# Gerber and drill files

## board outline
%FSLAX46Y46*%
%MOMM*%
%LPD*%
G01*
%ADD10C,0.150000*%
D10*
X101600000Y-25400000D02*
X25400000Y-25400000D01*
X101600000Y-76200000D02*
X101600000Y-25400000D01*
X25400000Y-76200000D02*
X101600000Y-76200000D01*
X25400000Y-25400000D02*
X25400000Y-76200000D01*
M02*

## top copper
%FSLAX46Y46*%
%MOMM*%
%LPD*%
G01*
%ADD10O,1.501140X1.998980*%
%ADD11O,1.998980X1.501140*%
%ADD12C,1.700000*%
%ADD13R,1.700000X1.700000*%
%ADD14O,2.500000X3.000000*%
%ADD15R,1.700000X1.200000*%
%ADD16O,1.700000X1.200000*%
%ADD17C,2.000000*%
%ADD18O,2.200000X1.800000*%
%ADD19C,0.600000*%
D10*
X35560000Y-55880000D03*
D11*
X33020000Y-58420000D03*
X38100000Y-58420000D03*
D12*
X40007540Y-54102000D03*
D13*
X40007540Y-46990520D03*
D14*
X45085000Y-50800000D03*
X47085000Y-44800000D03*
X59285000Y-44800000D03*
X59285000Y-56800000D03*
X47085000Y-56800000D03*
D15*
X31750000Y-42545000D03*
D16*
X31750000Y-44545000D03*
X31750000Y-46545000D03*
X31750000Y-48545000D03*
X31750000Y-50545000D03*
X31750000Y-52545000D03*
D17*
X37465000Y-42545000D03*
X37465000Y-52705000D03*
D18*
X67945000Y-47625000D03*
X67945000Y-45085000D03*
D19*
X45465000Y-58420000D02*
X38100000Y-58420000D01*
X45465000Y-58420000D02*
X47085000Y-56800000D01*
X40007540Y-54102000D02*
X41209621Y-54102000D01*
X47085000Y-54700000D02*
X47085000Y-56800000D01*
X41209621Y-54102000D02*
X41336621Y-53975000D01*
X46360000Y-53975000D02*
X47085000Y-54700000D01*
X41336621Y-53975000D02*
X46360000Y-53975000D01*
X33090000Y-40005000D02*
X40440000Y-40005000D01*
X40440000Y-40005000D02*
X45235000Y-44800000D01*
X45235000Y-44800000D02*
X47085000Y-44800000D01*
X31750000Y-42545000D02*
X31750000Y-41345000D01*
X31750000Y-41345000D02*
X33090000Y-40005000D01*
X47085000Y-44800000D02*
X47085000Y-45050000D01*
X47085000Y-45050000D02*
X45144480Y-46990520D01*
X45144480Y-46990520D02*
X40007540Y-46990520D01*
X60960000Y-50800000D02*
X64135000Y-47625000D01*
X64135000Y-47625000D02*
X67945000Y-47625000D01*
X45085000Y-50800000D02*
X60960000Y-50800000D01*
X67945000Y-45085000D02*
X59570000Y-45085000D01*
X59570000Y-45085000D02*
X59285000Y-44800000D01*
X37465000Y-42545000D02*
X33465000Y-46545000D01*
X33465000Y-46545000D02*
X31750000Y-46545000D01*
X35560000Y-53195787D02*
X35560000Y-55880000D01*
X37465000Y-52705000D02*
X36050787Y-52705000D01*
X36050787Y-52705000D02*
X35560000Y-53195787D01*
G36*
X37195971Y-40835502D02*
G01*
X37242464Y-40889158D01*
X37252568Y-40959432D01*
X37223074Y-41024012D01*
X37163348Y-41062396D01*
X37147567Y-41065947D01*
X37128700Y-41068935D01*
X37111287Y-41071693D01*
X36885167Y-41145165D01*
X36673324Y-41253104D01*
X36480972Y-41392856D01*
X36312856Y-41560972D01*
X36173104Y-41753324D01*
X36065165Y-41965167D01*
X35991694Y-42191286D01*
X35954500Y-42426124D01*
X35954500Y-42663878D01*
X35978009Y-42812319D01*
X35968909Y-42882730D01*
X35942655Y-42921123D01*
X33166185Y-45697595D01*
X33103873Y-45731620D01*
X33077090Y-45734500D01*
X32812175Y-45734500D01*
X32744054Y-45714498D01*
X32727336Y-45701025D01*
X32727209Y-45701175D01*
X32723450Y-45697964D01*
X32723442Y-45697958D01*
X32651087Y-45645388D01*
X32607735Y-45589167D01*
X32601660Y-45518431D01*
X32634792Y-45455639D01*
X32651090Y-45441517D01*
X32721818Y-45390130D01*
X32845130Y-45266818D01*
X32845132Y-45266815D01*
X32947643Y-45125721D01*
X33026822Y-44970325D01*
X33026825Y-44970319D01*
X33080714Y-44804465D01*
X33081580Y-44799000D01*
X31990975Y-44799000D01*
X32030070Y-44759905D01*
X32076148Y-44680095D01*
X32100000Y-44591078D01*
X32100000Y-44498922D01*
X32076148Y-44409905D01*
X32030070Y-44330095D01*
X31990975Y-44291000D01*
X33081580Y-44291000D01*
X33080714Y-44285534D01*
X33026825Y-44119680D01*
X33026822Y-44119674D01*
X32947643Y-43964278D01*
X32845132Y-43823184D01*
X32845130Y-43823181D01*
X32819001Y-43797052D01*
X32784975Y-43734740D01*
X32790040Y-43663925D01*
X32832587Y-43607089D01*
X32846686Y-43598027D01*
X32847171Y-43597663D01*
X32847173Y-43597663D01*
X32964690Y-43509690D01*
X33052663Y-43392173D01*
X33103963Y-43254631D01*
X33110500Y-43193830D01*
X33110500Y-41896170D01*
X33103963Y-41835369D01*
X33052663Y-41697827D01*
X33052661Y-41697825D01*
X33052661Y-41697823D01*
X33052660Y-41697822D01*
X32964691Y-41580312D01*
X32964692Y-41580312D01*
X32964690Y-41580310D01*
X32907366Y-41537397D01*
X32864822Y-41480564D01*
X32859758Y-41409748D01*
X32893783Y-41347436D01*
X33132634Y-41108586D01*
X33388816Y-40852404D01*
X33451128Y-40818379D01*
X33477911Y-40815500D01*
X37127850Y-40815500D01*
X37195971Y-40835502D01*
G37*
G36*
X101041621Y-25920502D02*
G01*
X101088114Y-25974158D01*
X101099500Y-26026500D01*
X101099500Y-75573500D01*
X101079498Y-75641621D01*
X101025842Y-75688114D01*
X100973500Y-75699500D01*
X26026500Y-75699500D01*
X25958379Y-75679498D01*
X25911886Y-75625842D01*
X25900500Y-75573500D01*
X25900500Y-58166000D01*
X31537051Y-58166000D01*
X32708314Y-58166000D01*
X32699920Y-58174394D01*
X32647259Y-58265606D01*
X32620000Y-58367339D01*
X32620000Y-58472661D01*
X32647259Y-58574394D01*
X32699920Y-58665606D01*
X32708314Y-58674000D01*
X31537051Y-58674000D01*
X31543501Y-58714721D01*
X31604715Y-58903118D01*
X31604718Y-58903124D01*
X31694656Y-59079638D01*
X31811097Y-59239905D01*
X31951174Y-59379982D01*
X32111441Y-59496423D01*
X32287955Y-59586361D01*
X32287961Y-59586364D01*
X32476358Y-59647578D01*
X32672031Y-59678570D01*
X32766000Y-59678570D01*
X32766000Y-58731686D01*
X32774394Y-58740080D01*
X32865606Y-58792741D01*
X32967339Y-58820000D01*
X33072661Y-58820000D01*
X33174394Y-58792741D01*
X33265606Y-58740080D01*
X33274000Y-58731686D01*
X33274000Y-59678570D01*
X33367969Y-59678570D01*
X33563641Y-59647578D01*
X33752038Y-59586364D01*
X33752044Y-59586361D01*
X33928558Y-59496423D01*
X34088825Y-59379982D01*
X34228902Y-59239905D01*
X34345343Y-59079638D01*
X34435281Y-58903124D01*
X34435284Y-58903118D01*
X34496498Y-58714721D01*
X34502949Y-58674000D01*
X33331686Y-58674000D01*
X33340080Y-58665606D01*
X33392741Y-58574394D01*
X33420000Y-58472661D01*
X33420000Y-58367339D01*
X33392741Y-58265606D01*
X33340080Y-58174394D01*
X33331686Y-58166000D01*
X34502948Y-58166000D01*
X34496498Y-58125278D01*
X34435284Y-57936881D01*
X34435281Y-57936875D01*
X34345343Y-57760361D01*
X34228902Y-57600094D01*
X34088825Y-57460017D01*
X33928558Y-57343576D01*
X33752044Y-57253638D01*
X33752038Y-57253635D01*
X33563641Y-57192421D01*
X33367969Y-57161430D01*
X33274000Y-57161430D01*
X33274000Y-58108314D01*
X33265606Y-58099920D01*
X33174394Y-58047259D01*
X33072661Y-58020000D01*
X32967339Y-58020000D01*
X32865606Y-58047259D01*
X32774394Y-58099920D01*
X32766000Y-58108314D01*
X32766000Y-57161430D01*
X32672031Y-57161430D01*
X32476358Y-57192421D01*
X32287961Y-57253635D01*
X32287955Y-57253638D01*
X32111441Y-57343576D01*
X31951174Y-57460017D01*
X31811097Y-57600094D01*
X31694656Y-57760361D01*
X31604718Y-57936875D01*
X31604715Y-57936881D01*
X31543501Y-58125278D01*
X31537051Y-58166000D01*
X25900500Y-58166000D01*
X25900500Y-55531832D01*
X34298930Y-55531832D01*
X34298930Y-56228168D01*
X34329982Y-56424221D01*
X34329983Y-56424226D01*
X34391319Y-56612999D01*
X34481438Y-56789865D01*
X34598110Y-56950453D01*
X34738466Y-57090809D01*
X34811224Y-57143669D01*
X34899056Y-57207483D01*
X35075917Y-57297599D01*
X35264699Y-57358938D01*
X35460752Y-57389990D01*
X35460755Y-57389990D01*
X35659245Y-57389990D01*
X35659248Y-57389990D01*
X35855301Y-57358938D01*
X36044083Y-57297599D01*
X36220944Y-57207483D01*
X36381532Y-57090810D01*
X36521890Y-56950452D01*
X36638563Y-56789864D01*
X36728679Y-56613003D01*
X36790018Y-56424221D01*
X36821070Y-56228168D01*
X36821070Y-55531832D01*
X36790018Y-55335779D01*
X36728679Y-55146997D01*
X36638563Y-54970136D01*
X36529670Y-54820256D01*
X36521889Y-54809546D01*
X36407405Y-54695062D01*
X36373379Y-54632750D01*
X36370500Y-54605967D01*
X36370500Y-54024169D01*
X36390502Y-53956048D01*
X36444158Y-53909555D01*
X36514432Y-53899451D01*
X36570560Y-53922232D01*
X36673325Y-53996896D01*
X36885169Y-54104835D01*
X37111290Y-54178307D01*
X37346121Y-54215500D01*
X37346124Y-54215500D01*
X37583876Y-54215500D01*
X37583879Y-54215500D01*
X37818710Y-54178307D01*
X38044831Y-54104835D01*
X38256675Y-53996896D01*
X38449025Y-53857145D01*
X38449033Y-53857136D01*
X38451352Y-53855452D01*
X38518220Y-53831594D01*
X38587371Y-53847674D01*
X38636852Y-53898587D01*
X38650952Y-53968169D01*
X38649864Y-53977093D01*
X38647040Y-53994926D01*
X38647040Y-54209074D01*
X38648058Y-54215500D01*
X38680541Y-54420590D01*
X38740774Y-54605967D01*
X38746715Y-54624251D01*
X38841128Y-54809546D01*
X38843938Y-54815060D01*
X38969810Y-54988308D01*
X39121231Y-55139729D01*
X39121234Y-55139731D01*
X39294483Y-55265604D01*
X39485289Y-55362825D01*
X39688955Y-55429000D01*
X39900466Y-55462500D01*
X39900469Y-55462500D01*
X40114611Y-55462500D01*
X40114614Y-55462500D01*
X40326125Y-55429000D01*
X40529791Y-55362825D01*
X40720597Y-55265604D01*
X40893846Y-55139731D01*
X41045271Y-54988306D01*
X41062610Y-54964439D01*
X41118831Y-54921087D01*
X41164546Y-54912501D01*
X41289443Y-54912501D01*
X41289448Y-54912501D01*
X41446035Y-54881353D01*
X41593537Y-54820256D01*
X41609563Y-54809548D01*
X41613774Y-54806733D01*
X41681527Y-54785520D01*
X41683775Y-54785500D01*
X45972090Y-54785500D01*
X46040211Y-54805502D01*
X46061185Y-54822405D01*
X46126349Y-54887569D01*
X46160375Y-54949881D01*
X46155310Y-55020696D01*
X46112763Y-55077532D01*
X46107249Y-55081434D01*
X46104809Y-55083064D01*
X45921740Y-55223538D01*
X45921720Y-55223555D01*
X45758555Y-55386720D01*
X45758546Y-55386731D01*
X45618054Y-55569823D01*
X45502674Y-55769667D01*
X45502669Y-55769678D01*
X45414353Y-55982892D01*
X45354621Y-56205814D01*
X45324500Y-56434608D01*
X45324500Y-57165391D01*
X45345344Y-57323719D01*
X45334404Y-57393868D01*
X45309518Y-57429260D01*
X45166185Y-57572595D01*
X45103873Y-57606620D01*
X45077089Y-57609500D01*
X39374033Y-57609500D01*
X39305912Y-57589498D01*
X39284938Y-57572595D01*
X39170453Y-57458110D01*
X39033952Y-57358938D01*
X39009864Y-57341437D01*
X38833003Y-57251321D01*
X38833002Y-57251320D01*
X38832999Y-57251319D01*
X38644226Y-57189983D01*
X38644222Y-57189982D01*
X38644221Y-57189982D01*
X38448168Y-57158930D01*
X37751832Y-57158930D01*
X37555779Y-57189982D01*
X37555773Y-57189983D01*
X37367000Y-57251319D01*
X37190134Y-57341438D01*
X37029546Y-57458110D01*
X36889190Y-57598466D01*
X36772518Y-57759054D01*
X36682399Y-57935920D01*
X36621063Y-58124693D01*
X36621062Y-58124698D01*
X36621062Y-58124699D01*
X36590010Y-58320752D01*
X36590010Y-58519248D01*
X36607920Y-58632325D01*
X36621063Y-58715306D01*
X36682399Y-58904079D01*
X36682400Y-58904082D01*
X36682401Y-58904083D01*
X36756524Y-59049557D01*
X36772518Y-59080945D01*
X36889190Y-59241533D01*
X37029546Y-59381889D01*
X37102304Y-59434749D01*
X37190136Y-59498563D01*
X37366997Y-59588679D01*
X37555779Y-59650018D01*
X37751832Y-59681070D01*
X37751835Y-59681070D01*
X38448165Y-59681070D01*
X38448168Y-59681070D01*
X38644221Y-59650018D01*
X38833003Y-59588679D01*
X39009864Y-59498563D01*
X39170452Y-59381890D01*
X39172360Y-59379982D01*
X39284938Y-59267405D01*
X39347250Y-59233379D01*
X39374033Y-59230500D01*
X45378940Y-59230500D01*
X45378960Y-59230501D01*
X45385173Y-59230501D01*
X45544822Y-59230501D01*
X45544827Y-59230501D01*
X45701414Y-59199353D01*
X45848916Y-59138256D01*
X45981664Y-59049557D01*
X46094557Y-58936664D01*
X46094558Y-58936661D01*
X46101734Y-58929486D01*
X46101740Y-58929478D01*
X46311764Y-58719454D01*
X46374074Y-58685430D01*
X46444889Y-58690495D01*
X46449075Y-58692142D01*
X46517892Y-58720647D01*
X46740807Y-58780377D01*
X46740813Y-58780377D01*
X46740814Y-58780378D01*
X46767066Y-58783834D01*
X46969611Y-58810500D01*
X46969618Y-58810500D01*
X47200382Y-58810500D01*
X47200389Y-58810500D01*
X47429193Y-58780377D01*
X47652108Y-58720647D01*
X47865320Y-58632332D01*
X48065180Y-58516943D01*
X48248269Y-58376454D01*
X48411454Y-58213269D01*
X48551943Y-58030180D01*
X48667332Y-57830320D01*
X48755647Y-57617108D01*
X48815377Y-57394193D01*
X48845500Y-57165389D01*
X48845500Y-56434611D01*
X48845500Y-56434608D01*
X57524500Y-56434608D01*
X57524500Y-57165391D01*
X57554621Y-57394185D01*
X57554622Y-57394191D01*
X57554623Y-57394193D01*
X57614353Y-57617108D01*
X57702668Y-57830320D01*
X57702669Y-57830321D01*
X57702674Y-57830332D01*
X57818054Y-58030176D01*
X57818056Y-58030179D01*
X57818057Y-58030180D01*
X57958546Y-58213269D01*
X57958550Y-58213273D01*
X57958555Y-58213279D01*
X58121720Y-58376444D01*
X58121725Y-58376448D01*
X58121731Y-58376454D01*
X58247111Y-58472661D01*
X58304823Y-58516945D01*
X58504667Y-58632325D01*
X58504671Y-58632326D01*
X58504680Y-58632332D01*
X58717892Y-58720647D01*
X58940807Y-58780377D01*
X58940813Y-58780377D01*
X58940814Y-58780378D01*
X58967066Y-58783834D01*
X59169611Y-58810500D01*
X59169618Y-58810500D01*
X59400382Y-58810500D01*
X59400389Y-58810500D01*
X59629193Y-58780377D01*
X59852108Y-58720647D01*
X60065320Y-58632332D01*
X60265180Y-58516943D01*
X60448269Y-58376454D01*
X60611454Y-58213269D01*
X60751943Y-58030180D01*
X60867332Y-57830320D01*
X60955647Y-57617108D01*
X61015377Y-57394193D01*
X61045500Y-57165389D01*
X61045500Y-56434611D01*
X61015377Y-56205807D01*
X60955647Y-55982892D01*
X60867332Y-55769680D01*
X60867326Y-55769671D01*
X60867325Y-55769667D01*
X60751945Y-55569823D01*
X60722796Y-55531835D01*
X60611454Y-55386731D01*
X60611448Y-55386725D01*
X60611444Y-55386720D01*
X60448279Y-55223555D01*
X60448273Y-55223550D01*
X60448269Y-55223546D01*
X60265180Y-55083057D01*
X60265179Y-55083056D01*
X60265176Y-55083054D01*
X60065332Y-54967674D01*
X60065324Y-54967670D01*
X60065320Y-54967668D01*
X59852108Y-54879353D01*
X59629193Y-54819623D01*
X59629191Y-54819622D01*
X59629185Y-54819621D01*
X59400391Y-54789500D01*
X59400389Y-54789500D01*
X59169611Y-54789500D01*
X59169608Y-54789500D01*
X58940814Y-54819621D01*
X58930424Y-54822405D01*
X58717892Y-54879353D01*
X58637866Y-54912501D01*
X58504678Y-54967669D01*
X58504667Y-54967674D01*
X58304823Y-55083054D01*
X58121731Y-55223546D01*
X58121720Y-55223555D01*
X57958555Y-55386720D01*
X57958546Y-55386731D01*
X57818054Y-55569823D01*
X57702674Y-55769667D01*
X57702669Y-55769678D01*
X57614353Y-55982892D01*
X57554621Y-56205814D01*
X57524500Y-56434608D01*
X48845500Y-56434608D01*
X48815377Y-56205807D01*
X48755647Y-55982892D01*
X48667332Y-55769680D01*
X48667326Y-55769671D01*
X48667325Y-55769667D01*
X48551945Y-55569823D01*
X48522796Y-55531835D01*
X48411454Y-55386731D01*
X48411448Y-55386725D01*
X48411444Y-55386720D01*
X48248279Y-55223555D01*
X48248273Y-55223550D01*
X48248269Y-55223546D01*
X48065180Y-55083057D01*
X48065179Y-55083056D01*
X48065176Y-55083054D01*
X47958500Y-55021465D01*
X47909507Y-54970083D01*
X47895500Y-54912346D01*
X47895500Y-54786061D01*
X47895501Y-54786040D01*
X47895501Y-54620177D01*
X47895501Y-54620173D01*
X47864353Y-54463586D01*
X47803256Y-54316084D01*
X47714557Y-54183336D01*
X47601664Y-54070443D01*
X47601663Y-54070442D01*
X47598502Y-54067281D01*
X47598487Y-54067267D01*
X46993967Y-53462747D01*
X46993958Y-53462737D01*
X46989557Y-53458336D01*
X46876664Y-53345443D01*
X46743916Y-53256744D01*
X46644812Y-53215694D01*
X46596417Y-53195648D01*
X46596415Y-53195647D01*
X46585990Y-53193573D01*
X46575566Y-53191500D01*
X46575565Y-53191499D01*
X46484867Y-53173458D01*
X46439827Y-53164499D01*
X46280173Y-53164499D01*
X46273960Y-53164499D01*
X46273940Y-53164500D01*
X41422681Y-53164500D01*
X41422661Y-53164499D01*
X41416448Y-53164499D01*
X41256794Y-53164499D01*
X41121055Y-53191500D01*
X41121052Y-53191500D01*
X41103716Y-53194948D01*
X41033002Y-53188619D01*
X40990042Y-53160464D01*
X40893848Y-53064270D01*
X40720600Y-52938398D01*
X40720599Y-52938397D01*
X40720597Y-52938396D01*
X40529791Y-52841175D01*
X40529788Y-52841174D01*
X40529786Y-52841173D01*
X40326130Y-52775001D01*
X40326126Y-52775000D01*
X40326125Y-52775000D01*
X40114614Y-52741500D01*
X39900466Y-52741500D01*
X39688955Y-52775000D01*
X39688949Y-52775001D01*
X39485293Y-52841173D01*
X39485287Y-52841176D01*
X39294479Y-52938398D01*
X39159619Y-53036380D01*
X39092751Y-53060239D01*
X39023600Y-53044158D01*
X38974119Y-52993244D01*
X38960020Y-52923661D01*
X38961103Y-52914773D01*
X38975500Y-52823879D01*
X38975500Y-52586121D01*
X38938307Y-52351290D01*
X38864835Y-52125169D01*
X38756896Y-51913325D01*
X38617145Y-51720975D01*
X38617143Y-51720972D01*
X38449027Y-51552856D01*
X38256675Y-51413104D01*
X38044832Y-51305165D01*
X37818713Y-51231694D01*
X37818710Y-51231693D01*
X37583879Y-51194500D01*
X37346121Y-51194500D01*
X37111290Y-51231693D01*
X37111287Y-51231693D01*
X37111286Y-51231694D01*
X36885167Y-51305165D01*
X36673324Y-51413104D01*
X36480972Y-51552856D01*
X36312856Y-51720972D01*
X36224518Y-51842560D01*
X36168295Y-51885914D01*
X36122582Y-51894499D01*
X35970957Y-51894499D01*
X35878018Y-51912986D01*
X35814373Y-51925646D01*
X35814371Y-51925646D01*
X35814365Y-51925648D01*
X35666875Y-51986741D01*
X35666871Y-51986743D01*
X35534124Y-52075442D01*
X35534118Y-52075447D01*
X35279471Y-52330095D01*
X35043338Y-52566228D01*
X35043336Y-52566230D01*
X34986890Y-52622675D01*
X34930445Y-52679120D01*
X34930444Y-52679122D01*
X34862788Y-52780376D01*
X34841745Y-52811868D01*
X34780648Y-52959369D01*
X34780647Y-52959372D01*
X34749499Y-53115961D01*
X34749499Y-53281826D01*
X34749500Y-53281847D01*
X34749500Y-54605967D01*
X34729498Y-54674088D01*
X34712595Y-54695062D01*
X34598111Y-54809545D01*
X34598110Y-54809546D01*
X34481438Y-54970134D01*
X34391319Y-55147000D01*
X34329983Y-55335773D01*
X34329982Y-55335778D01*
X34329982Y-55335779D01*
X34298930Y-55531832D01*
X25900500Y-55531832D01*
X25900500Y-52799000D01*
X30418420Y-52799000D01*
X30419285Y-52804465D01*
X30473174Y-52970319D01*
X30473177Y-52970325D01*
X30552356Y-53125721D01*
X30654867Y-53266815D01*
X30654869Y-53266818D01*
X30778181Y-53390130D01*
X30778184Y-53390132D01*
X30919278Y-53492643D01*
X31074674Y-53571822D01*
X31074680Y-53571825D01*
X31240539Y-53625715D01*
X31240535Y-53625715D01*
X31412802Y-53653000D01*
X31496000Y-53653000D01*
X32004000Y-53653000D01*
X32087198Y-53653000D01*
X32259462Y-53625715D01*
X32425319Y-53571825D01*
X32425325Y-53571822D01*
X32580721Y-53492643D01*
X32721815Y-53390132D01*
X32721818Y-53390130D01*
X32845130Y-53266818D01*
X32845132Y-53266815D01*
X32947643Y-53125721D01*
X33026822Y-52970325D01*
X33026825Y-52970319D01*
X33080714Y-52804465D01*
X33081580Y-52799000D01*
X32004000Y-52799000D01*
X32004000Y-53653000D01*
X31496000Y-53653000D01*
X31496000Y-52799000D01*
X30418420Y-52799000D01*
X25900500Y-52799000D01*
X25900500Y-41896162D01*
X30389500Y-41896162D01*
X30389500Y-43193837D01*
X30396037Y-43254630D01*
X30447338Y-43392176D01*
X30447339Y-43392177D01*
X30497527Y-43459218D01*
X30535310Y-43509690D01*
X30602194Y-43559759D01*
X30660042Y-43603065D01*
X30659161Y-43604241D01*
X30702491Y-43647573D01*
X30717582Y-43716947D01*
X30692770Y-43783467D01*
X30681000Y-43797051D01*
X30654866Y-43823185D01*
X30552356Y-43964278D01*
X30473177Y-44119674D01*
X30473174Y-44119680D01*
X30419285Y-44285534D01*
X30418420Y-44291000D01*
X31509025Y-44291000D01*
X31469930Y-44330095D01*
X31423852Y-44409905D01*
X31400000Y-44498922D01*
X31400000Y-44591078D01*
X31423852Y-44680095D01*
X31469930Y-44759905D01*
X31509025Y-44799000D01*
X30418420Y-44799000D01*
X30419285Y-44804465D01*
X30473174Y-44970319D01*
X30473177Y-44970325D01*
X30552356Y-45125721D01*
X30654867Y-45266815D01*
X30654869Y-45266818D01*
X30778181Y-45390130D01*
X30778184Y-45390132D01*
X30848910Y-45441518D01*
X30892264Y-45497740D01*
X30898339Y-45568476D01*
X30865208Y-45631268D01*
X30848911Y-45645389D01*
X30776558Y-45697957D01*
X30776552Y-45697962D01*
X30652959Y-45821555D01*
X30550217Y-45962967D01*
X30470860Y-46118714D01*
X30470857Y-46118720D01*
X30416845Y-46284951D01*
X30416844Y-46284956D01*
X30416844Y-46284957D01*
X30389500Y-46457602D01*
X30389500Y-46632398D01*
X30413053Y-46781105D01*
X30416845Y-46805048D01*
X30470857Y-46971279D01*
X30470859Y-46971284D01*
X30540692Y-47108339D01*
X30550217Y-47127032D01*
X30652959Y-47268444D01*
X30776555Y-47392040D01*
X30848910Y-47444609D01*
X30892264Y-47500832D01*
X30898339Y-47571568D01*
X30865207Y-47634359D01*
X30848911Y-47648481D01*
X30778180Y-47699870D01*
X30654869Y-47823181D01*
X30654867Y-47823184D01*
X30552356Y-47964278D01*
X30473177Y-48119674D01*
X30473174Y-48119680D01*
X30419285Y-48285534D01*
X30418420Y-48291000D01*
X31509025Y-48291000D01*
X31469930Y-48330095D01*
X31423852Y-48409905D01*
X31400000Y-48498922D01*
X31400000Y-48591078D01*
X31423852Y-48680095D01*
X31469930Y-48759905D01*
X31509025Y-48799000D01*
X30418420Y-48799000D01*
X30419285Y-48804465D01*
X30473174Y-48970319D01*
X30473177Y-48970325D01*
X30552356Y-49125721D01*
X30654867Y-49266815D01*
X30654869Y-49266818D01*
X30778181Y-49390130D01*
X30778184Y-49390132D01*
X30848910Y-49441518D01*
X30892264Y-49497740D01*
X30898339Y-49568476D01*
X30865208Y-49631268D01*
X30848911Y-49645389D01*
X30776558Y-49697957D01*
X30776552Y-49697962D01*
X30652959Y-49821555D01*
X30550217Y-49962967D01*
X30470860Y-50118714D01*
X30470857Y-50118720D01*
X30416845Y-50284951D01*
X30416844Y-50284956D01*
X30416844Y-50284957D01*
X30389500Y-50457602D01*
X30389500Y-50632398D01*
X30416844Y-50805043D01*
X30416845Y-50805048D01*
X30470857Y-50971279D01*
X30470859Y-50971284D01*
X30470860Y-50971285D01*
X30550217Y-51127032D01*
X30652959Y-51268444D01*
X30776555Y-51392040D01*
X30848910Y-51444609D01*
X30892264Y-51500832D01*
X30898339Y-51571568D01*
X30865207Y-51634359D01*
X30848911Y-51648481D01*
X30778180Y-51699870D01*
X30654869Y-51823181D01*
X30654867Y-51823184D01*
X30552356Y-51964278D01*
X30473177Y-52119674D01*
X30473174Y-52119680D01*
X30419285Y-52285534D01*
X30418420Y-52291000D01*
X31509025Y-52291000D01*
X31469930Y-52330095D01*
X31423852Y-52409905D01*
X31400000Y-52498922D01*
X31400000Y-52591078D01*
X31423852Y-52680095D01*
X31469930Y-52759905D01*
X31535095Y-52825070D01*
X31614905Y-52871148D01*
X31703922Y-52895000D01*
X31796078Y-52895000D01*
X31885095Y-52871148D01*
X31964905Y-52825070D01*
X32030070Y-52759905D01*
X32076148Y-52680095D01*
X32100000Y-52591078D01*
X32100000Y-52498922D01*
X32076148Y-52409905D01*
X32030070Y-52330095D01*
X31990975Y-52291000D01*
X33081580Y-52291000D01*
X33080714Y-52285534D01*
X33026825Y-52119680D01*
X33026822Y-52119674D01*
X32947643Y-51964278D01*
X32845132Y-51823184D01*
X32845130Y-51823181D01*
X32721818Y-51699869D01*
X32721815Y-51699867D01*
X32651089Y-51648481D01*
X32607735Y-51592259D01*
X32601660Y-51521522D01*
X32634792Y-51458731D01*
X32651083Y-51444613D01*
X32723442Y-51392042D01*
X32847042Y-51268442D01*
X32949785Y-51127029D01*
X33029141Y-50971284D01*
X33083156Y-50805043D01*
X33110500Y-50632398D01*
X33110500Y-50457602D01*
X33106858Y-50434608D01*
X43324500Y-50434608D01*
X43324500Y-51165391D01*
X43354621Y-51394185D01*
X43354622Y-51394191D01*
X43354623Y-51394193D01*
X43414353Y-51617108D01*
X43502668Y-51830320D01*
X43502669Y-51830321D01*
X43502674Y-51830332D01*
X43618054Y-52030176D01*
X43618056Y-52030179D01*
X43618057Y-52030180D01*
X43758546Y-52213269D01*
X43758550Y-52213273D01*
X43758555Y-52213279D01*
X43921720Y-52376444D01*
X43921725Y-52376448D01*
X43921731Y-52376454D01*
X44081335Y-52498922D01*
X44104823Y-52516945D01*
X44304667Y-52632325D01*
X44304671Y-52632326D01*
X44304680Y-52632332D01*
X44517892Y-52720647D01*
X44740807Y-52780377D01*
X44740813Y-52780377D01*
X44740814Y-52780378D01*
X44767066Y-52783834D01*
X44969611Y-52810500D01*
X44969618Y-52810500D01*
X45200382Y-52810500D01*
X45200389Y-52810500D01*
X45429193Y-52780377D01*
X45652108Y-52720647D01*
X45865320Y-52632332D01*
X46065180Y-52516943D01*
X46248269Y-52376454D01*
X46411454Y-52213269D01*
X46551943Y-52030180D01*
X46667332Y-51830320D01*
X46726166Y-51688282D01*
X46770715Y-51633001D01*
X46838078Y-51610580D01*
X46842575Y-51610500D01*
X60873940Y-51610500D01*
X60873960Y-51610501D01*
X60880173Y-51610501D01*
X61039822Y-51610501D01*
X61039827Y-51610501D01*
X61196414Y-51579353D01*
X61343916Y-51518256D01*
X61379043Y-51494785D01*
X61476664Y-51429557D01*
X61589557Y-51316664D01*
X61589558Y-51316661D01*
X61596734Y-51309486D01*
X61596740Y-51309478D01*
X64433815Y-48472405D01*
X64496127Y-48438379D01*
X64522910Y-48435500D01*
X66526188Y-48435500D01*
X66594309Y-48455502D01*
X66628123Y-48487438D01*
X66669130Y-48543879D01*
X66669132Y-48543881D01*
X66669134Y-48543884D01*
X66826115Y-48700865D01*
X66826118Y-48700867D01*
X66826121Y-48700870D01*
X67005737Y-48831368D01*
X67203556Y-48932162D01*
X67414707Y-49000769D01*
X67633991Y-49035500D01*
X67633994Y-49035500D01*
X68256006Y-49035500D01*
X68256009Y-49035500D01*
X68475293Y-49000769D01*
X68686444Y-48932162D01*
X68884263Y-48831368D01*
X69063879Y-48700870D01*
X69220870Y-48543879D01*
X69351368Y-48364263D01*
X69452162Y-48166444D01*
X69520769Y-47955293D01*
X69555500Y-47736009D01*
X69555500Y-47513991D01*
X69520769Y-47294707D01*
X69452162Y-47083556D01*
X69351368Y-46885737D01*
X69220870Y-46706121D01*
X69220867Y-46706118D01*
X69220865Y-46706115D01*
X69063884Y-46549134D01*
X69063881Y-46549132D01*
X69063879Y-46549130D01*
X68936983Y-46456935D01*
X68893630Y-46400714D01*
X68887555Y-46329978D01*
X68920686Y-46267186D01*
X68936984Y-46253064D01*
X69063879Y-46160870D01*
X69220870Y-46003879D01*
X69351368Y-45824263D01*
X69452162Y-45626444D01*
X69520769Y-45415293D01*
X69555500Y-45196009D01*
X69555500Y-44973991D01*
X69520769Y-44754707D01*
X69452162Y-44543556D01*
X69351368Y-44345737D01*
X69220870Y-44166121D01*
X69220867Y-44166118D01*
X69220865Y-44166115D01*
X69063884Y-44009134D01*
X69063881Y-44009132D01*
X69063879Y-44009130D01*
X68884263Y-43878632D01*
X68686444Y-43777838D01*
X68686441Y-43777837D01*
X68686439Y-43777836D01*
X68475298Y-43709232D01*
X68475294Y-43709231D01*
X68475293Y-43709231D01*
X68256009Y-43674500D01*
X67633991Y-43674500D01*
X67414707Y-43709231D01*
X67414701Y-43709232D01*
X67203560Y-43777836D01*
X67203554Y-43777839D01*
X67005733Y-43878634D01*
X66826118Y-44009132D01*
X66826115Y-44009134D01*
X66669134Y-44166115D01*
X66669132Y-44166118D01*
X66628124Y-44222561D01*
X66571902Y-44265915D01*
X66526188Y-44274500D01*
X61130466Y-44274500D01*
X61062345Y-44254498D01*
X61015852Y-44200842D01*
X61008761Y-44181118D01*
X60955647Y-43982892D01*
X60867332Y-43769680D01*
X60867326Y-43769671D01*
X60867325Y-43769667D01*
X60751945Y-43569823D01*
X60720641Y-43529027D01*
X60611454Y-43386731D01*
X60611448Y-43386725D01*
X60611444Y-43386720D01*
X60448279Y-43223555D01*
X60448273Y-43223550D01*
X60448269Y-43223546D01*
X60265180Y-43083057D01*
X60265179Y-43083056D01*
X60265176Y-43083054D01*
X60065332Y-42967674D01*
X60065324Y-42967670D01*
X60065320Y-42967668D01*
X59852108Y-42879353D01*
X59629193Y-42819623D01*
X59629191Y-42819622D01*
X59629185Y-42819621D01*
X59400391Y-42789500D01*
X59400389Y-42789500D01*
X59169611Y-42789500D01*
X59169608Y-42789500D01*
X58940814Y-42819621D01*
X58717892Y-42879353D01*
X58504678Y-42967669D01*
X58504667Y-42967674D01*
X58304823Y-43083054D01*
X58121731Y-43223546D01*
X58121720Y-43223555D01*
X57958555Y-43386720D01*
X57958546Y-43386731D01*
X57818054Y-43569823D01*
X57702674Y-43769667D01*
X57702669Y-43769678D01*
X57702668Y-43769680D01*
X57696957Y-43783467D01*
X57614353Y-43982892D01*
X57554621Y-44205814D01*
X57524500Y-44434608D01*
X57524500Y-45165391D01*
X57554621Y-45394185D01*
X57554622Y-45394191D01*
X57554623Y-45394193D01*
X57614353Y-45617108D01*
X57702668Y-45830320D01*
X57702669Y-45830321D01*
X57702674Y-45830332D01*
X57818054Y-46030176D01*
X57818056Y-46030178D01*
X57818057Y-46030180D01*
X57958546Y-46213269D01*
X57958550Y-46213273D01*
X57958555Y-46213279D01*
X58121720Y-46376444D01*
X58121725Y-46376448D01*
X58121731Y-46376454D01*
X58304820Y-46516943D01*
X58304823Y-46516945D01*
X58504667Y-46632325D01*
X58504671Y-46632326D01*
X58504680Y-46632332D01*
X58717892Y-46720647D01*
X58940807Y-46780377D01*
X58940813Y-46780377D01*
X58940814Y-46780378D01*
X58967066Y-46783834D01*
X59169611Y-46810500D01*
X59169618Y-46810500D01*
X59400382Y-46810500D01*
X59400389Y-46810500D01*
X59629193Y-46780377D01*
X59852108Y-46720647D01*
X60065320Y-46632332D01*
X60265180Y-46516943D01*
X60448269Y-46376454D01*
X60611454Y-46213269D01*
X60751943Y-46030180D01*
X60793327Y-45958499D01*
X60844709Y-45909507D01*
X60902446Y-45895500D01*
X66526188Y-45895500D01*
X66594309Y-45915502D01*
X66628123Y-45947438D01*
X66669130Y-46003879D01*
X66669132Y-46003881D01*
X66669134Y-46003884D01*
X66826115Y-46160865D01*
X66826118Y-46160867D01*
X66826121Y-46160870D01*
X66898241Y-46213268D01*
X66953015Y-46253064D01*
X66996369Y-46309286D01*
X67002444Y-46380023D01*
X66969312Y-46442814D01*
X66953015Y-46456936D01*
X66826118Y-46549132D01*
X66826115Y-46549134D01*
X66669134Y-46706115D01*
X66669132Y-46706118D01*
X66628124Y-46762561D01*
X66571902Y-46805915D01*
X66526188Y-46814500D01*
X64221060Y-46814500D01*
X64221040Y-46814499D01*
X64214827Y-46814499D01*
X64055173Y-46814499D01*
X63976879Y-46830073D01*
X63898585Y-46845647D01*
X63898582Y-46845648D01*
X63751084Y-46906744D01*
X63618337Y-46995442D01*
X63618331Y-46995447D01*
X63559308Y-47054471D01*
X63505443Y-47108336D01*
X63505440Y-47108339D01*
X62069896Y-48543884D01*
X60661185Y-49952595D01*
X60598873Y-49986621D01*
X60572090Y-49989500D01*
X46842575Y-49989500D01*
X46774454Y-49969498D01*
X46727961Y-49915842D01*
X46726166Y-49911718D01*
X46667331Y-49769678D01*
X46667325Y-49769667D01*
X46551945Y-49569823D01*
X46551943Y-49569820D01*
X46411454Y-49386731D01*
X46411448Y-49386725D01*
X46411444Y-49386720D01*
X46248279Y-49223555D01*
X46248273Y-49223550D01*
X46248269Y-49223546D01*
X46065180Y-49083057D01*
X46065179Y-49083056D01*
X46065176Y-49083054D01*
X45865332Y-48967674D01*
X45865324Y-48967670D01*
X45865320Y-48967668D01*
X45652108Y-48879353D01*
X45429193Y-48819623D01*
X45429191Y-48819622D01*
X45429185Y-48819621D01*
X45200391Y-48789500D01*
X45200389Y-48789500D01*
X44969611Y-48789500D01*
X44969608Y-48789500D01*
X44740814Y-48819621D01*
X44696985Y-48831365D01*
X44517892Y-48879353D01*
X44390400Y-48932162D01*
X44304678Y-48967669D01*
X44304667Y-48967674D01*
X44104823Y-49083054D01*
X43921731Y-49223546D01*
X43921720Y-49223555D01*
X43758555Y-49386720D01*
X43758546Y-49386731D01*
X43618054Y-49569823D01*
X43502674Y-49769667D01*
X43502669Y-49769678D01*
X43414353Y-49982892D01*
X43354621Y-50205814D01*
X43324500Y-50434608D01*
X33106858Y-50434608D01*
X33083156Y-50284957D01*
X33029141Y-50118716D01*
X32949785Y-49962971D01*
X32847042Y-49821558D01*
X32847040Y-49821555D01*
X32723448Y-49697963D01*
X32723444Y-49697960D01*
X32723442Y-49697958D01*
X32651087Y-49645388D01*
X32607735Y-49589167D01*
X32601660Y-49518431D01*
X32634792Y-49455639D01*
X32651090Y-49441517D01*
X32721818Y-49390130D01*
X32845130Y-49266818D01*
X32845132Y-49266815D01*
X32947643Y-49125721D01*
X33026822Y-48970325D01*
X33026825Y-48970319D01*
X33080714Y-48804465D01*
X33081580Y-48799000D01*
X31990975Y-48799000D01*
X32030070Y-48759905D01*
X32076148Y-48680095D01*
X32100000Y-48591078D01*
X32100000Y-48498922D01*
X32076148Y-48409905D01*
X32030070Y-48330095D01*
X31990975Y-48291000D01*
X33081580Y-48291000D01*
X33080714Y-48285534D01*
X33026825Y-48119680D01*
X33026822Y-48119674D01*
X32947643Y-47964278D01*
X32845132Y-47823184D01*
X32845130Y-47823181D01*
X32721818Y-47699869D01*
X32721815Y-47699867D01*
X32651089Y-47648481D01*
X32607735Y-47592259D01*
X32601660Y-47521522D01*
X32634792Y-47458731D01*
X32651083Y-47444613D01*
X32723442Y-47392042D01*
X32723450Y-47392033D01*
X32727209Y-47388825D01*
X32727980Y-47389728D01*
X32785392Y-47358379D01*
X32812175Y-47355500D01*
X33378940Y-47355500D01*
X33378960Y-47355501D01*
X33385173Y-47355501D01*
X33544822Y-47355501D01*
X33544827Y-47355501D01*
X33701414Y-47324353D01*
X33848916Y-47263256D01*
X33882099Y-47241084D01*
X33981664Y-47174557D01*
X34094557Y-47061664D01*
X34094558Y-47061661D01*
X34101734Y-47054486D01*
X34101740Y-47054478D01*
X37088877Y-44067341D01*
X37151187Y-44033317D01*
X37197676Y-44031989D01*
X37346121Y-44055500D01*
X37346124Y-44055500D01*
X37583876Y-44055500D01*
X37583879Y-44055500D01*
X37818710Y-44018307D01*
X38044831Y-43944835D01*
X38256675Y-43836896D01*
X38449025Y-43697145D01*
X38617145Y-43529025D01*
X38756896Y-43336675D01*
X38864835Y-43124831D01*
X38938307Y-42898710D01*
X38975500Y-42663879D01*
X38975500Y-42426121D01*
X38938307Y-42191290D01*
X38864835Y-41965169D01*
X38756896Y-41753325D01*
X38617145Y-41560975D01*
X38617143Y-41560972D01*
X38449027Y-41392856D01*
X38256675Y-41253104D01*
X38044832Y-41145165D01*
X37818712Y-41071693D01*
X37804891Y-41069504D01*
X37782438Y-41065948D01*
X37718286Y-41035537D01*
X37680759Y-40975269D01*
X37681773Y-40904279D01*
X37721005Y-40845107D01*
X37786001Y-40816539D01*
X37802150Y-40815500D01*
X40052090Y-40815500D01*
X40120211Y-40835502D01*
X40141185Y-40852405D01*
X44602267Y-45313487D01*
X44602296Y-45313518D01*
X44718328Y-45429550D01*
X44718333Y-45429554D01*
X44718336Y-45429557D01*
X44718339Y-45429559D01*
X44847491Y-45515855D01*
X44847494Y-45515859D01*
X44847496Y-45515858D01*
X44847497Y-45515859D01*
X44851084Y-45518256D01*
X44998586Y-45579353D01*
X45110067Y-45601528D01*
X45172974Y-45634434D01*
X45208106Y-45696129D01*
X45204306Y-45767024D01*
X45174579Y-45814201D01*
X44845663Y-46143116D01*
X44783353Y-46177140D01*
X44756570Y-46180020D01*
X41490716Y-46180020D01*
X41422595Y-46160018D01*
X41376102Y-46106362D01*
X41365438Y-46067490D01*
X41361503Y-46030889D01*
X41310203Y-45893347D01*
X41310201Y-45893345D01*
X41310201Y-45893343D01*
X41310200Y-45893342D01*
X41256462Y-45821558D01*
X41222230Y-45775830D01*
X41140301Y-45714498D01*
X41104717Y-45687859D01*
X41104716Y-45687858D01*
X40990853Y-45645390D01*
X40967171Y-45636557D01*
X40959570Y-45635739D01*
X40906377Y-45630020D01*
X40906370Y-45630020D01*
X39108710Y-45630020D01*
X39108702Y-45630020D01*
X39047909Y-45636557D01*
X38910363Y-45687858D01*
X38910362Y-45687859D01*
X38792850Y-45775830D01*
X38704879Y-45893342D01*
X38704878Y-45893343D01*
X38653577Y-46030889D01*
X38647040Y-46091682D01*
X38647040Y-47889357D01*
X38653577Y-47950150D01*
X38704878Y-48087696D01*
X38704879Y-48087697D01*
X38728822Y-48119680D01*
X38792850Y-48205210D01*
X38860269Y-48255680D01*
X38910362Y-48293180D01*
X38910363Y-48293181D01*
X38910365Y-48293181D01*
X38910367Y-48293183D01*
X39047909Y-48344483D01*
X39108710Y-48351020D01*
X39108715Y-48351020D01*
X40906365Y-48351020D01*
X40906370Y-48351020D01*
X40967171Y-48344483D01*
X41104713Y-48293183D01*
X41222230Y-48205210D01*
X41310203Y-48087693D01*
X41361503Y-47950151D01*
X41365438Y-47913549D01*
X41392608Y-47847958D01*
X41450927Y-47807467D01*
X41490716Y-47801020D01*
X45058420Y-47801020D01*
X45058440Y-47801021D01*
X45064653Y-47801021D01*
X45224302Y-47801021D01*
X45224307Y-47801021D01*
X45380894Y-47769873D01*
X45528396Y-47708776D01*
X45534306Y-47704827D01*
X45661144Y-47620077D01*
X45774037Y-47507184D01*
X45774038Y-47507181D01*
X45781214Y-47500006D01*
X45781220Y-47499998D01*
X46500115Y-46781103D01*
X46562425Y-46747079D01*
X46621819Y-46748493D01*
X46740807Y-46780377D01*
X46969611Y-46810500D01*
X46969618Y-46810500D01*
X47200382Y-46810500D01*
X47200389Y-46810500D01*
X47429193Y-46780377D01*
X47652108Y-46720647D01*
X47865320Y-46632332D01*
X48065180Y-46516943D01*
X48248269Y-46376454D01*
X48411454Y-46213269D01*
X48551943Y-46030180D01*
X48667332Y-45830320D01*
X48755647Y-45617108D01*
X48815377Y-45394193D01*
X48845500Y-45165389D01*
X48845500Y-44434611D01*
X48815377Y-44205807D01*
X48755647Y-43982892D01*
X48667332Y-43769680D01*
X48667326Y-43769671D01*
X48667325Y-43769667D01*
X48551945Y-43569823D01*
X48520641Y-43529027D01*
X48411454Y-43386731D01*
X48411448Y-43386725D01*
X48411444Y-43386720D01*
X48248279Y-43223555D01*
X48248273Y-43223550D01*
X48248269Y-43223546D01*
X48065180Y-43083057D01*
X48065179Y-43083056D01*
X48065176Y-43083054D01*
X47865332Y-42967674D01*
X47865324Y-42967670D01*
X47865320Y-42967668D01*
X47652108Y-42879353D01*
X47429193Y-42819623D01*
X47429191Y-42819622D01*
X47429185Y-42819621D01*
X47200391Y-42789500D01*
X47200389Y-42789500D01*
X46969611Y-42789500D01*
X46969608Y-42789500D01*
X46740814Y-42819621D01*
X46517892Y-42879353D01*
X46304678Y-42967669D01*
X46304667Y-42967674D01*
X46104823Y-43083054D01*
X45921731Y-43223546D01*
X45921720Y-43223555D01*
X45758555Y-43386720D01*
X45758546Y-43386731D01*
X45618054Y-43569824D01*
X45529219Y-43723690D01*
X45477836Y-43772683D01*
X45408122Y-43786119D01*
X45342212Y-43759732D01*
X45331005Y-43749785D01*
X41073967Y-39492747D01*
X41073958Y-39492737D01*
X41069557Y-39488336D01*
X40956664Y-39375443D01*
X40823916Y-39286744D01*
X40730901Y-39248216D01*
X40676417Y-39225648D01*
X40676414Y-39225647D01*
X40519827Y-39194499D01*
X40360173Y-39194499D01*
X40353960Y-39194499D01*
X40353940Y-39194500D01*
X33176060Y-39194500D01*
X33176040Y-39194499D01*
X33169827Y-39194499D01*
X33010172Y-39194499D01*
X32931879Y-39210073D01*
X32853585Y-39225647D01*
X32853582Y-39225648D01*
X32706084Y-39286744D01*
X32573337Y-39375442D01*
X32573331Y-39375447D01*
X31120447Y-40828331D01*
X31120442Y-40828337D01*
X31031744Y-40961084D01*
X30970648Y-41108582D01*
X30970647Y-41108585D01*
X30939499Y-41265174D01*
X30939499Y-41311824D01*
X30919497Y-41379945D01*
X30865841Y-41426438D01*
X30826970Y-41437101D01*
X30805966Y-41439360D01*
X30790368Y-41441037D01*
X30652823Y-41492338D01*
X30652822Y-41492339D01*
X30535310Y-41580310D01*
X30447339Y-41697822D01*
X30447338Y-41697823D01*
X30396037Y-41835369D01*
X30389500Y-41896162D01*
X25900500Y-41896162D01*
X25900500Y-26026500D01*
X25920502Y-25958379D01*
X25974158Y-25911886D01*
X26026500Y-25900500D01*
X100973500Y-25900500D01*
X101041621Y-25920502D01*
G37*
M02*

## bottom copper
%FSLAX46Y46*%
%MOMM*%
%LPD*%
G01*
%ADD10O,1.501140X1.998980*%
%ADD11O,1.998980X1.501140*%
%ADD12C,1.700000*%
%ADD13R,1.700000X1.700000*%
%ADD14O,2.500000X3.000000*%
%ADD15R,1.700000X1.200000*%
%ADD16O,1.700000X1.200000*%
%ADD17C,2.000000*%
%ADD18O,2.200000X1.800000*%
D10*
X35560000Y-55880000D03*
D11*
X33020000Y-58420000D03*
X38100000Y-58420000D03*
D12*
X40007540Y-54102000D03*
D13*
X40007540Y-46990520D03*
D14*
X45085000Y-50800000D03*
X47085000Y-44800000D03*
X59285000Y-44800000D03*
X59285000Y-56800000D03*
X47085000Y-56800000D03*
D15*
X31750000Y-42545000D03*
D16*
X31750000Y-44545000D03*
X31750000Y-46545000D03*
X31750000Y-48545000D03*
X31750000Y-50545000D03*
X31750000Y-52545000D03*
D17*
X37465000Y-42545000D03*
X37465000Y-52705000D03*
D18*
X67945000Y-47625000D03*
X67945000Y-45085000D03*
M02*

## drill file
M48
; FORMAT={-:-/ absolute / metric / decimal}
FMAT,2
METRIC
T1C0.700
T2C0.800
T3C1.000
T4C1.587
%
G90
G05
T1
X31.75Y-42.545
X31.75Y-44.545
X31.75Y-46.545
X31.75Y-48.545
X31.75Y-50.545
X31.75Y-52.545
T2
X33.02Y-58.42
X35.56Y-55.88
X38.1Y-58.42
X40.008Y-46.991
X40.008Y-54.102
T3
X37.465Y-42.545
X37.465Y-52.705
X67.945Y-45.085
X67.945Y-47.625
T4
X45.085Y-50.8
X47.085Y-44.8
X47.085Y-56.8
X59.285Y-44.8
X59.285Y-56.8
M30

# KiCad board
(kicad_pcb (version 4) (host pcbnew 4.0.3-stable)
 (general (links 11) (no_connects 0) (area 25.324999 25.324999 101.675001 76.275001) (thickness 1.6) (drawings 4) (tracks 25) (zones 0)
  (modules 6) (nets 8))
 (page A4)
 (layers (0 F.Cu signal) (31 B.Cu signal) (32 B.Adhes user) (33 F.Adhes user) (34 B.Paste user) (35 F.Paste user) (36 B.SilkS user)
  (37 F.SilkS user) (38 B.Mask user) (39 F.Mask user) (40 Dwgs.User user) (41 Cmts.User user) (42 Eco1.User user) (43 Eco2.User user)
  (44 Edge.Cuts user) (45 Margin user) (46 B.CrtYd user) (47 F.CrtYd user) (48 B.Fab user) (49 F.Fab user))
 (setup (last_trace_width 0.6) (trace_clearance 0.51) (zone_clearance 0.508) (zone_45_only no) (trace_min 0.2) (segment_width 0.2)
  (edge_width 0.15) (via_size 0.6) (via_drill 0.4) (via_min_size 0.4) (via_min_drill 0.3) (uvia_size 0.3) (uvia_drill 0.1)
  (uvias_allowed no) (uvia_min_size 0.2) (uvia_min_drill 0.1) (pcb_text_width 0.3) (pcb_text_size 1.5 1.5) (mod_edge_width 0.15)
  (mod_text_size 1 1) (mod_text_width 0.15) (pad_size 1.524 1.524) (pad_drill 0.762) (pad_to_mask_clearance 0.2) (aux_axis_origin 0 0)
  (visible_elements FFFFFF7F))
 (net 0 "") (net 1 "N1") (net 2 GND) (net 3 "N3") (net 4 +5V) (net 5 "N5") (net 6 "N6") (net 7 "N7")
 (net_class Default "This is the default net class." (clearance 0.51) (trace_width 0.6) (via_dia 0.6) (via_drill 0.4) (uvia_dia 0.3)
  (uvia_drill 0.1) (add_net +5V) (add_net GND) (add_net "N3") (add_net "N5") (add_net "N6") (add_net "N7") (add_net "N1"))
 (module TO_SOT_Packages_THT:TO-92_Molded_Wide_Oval (layer F.Cu) (at 33.02 58.42)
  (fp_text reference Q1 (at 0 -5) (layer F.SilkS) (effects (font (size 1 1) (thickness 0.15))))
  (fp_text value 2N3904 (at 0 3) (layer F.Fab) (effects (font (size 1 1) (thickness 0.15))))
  (pad 2 thru_hole oval (at 2.54 -2.54 90) (size 1.99898 1.50114) (drill 0.8) (layers *.Cu *.Mask F.SilkS) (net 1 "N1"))
  (pad 1 thru_hole oval (at 0 0 90) (size 1.50114 1.99898) (drill 0.8) (layers *.Cu *.Mask F.SilkS) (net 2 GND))
  (pad 3 thru_hole oval (at 5.08 0 90) (size 1.50114 1.99898) (drill 0.8) (layers *.Cu *.Mask F.SilkS) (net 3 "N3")))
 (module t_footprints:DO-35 (layer F.Cu) (at 40.005 46.99 270)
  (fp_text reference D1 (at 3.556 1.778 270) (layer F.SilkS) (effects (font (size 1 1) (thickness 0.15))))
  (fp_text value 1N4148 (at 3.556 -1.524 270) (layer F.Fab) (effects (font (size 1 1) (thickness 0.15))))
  (pad 2 thru_hole circle (at 7.112 -0.00254 90) (size 1.7 1.7) (drill 0.8) (layers *.Cu *.Mask F.SilkS) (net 3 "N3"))
  (pad 1 thru_hole rect (at 0.00052 -0.00254 90) (size 1.7 1.7) (drill 0.8) (layers *.Cu *.Mask F.SilkS) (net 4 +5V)))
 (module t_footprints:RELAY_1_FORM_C (layer F.Cu) (at 45.085 50.8)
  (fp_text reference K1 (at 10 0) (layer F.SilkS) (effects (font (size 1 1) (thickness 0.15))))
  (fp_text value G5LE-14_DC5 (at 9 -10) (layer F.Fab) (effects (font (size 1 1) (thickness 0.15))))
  (pad 1 thru_hole oval (at 0 0) (size 2.5 3) (drill 1.5875) (layers *.Cu *.Mask) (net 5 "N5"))
  (pad 2 thru_hole oval (at 2 -6) (size 2.5 3) (drill 1.5875) (layers *.Cu *.Mask) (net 4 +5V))
  (pad 3 thru_hole oval (at 14.2 -6) (size 2.5 3) (drill 1.5875) (layers *.Cu *.Mask) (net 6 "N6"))
  (pad 4 thru_hole oval (at 14.2 6) (size 2.5 3) (drill 1.5875) (layers *.Cu *.Mask))
  (pad 5 thru_hole oval (at 2 6) (size 2.5 3) (drill 1.5875) (layers *.Cu *.Mask) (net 3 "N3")))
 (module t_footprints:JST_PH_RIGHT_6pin (layer F.Cu) (at 31.75 42.545 270)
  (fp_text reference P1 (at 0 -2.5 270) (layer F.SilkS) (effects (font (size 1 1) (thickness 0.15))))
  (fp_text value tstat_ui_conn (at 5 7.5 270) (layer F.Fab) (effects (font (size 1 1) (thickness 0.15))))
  (pad 1 thru_hole rect (at 0 0 270) (size 1.2 1.7) (drill 0.7) (layers *.Cu *.Mask F.SilkS) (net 4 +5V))
  (pad 2 thru_hole oval (at 2 0 270) (size 1.2 1.7) (drill 0.7) (layers *.Cu *.Mask F.SilkS) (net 2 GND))
  (pad 3 thru_hole oval (at 4 0 270) (size 1.2 1.7) (drill 0.7) (layers *.Cu *.Mask F.SilkS) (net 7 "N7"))
  (pad 4 thru_hole oval (at 6 0 270) (size 1.2 1.7) (drill 0.7) (layers *.Cu *.Mask F.SilkS) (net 2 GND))
  (pad 5 thru_hole oval (at 8 0 270) (size 1.2 1.7) (drill 0.7) (layers *.Cu *.Mask F.SilkS))
  (pad 6 thru_hole oval (at 10 0 270) (size 1.2 1.7) (drill 0.7) (layers *.Cu *.Mask F.SilkS) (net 2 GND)))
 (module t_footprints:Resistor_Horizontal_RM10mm (layer F.Cu) (at 37.465 42.545 270)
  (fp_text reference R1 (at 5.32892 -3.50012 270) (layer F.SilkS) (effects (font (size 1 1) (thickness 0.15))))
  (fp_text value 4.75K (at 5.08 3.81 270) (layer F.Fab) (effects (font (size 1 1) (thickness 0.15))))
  (pad 1 thru_hole circle (at 0 0 270) (size 2 2) (drill 1) (layers *.Cu *.SilkS *.Mask) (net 7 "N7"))
  (pad 2 thru_hole circle (at 10.16 0 270) (size 2 2) (drill 1) (layers *.Cu *.SilkS *.Mask) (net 1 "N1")))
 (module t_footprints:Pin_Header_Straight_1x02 (layer F.Cu) (at 67.945 47.625 180)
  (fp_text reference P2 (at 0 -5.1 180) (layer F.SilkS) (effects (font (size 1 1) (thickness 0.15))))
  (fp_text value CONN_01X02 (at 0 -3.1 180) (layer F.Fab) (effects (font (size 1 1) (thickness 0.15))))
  (pad 1 thru_hole oval (at 0 0 180) (size 2.2 1.8) (drill 1) (layers *.Cu *.Mask F.SilkS) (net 5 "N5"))
  (pad 2 thru_hole oval (at 0 2.54 180) (size 2.2 1.8) (drill 1) (layers *.Cu *.Mask F.SilkS) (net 6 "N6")))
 (gr_line (start 101.6 25.4) (end 25.4 25.4) (angle 90) (layer Edge.Cuts) (width 0.15))
 (gr_line (start 101.6 76.2) (end 101.6 25.4) (angle 90) (layer Edge.Cuts) (width 0.15))
 (gr_line (start 25.4 76.2) (end 101.6 76.2) (angle 90) (layer Edge.Cuts) (width 0.15))
 (gr_line (start 25.4 25.4) (end 25.4 76.2) (angle 90) (layer Edge.Cuts) (width 0.15))
 (segment (start 45.465 58.42) (end 38.1 58.42) (width 0.6) (layer F.Cu) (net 3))
 (segment (start 45.465 58.42) (end 47.085 56.8) (width 0.6) (layer F.Cu) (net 3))
 (segment (start 40.00754 54.102) (end 41.209621 54.102) (width 0.6) (layer F.Cu) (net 3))
 (segment (start 47.085 54.7) (end 47.085 56.8) (width 0.6) (layer F.Cu) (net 3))
 (segment (start 41.209621 54.102) (end 41.336621 53.975) (width 0.6) (layer F.Cu) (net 3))
 (segment (start 46.36 53.975) (end 47.085 54.7) (width 0.6) (layer F.Cu) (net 3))
 (segment (start 41.336621 53.975) (end 46.36 53.975) (width 0.6) (layer F.Cu) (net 3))
 (segment (start 33.09 40.005) (end 40.44 40.005) (width 0.6) (layer F.Cu) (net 4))
 (segment (start 40.44 40.005) (end 45.235 44.8) (width 0.6) (layer F.Cu) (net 4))
 (segment (start 45.235 44.8) (end 47.085 44.8) (width 0.6) (layer F.Cu) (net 4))
 (segment (start 31.75 42.545) (end 31.75 41.345) (width 0.6) (layer F.Cu) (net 4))
 (segment (start 31.75 41.345) (end 33.09 40.005) (width 0.6) (layer F.Cu) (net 4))
 (segment (start 47.085 44.8) (end 47.085 45.05) (width 0.6) (layer F.Cu) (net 4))
 (segment (start 47.085 45.05) (end 45.14448 46.99052) (width 0.6) (layer F.Cu) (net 4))
 (segment (start 45.14448 46.99052) (end 40.00754 46.99052) (width 0.6) (layer F.Cu) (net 4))
 (segment (start 60.96 50.8) (end 64.135 47.625) (width 0.6) (layer F.Cu) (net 5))
 (segment (start 64.135 47.625) (end 67.945 47.625) (width 0.6) (layer F.Cu) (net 5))
 (segment (start 45.085 50.8) (end 60.96 50.8) (width 0.6) (layer F.Cu) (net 5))
 (segment (start 67.945 45.085) (end 59.57 45.085) (width 0.6) (layer F.Cu) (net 6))
 (segment (start 59.57 45.085) (end 59.285 44.8) (width 0.6) (layer F.Cu) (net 6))
 (segment (start 37.465 42.545) (end 33.465 46.545) (width 0.6) (layer F.Cu) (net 7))
 (segment (start 33.465 46.545) (end 31.75 46.545) (width 0.6) (layer F.Cu) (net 7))
 (segment (start 35.56 53.195787) (end 35.56 55.88) (width 0.6) (layer F.Cu) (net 1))
 (segment (start 37.465 52.705) (end 36.050787 52.705) (width 0.6) (layer F.Cu) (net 1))
 (segment (start 36.050787 52.705) (end 35.56 53.195787) (width 0.6) (layer F.Cu) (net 1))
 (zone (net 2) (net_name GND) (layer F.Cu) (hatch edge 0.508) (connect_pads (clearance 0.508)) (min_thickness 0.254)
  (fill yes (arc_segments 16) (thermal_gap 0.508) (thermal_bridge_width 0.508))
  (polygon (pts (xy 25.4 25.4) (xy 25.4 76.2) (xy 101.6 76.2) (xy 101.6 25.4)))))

